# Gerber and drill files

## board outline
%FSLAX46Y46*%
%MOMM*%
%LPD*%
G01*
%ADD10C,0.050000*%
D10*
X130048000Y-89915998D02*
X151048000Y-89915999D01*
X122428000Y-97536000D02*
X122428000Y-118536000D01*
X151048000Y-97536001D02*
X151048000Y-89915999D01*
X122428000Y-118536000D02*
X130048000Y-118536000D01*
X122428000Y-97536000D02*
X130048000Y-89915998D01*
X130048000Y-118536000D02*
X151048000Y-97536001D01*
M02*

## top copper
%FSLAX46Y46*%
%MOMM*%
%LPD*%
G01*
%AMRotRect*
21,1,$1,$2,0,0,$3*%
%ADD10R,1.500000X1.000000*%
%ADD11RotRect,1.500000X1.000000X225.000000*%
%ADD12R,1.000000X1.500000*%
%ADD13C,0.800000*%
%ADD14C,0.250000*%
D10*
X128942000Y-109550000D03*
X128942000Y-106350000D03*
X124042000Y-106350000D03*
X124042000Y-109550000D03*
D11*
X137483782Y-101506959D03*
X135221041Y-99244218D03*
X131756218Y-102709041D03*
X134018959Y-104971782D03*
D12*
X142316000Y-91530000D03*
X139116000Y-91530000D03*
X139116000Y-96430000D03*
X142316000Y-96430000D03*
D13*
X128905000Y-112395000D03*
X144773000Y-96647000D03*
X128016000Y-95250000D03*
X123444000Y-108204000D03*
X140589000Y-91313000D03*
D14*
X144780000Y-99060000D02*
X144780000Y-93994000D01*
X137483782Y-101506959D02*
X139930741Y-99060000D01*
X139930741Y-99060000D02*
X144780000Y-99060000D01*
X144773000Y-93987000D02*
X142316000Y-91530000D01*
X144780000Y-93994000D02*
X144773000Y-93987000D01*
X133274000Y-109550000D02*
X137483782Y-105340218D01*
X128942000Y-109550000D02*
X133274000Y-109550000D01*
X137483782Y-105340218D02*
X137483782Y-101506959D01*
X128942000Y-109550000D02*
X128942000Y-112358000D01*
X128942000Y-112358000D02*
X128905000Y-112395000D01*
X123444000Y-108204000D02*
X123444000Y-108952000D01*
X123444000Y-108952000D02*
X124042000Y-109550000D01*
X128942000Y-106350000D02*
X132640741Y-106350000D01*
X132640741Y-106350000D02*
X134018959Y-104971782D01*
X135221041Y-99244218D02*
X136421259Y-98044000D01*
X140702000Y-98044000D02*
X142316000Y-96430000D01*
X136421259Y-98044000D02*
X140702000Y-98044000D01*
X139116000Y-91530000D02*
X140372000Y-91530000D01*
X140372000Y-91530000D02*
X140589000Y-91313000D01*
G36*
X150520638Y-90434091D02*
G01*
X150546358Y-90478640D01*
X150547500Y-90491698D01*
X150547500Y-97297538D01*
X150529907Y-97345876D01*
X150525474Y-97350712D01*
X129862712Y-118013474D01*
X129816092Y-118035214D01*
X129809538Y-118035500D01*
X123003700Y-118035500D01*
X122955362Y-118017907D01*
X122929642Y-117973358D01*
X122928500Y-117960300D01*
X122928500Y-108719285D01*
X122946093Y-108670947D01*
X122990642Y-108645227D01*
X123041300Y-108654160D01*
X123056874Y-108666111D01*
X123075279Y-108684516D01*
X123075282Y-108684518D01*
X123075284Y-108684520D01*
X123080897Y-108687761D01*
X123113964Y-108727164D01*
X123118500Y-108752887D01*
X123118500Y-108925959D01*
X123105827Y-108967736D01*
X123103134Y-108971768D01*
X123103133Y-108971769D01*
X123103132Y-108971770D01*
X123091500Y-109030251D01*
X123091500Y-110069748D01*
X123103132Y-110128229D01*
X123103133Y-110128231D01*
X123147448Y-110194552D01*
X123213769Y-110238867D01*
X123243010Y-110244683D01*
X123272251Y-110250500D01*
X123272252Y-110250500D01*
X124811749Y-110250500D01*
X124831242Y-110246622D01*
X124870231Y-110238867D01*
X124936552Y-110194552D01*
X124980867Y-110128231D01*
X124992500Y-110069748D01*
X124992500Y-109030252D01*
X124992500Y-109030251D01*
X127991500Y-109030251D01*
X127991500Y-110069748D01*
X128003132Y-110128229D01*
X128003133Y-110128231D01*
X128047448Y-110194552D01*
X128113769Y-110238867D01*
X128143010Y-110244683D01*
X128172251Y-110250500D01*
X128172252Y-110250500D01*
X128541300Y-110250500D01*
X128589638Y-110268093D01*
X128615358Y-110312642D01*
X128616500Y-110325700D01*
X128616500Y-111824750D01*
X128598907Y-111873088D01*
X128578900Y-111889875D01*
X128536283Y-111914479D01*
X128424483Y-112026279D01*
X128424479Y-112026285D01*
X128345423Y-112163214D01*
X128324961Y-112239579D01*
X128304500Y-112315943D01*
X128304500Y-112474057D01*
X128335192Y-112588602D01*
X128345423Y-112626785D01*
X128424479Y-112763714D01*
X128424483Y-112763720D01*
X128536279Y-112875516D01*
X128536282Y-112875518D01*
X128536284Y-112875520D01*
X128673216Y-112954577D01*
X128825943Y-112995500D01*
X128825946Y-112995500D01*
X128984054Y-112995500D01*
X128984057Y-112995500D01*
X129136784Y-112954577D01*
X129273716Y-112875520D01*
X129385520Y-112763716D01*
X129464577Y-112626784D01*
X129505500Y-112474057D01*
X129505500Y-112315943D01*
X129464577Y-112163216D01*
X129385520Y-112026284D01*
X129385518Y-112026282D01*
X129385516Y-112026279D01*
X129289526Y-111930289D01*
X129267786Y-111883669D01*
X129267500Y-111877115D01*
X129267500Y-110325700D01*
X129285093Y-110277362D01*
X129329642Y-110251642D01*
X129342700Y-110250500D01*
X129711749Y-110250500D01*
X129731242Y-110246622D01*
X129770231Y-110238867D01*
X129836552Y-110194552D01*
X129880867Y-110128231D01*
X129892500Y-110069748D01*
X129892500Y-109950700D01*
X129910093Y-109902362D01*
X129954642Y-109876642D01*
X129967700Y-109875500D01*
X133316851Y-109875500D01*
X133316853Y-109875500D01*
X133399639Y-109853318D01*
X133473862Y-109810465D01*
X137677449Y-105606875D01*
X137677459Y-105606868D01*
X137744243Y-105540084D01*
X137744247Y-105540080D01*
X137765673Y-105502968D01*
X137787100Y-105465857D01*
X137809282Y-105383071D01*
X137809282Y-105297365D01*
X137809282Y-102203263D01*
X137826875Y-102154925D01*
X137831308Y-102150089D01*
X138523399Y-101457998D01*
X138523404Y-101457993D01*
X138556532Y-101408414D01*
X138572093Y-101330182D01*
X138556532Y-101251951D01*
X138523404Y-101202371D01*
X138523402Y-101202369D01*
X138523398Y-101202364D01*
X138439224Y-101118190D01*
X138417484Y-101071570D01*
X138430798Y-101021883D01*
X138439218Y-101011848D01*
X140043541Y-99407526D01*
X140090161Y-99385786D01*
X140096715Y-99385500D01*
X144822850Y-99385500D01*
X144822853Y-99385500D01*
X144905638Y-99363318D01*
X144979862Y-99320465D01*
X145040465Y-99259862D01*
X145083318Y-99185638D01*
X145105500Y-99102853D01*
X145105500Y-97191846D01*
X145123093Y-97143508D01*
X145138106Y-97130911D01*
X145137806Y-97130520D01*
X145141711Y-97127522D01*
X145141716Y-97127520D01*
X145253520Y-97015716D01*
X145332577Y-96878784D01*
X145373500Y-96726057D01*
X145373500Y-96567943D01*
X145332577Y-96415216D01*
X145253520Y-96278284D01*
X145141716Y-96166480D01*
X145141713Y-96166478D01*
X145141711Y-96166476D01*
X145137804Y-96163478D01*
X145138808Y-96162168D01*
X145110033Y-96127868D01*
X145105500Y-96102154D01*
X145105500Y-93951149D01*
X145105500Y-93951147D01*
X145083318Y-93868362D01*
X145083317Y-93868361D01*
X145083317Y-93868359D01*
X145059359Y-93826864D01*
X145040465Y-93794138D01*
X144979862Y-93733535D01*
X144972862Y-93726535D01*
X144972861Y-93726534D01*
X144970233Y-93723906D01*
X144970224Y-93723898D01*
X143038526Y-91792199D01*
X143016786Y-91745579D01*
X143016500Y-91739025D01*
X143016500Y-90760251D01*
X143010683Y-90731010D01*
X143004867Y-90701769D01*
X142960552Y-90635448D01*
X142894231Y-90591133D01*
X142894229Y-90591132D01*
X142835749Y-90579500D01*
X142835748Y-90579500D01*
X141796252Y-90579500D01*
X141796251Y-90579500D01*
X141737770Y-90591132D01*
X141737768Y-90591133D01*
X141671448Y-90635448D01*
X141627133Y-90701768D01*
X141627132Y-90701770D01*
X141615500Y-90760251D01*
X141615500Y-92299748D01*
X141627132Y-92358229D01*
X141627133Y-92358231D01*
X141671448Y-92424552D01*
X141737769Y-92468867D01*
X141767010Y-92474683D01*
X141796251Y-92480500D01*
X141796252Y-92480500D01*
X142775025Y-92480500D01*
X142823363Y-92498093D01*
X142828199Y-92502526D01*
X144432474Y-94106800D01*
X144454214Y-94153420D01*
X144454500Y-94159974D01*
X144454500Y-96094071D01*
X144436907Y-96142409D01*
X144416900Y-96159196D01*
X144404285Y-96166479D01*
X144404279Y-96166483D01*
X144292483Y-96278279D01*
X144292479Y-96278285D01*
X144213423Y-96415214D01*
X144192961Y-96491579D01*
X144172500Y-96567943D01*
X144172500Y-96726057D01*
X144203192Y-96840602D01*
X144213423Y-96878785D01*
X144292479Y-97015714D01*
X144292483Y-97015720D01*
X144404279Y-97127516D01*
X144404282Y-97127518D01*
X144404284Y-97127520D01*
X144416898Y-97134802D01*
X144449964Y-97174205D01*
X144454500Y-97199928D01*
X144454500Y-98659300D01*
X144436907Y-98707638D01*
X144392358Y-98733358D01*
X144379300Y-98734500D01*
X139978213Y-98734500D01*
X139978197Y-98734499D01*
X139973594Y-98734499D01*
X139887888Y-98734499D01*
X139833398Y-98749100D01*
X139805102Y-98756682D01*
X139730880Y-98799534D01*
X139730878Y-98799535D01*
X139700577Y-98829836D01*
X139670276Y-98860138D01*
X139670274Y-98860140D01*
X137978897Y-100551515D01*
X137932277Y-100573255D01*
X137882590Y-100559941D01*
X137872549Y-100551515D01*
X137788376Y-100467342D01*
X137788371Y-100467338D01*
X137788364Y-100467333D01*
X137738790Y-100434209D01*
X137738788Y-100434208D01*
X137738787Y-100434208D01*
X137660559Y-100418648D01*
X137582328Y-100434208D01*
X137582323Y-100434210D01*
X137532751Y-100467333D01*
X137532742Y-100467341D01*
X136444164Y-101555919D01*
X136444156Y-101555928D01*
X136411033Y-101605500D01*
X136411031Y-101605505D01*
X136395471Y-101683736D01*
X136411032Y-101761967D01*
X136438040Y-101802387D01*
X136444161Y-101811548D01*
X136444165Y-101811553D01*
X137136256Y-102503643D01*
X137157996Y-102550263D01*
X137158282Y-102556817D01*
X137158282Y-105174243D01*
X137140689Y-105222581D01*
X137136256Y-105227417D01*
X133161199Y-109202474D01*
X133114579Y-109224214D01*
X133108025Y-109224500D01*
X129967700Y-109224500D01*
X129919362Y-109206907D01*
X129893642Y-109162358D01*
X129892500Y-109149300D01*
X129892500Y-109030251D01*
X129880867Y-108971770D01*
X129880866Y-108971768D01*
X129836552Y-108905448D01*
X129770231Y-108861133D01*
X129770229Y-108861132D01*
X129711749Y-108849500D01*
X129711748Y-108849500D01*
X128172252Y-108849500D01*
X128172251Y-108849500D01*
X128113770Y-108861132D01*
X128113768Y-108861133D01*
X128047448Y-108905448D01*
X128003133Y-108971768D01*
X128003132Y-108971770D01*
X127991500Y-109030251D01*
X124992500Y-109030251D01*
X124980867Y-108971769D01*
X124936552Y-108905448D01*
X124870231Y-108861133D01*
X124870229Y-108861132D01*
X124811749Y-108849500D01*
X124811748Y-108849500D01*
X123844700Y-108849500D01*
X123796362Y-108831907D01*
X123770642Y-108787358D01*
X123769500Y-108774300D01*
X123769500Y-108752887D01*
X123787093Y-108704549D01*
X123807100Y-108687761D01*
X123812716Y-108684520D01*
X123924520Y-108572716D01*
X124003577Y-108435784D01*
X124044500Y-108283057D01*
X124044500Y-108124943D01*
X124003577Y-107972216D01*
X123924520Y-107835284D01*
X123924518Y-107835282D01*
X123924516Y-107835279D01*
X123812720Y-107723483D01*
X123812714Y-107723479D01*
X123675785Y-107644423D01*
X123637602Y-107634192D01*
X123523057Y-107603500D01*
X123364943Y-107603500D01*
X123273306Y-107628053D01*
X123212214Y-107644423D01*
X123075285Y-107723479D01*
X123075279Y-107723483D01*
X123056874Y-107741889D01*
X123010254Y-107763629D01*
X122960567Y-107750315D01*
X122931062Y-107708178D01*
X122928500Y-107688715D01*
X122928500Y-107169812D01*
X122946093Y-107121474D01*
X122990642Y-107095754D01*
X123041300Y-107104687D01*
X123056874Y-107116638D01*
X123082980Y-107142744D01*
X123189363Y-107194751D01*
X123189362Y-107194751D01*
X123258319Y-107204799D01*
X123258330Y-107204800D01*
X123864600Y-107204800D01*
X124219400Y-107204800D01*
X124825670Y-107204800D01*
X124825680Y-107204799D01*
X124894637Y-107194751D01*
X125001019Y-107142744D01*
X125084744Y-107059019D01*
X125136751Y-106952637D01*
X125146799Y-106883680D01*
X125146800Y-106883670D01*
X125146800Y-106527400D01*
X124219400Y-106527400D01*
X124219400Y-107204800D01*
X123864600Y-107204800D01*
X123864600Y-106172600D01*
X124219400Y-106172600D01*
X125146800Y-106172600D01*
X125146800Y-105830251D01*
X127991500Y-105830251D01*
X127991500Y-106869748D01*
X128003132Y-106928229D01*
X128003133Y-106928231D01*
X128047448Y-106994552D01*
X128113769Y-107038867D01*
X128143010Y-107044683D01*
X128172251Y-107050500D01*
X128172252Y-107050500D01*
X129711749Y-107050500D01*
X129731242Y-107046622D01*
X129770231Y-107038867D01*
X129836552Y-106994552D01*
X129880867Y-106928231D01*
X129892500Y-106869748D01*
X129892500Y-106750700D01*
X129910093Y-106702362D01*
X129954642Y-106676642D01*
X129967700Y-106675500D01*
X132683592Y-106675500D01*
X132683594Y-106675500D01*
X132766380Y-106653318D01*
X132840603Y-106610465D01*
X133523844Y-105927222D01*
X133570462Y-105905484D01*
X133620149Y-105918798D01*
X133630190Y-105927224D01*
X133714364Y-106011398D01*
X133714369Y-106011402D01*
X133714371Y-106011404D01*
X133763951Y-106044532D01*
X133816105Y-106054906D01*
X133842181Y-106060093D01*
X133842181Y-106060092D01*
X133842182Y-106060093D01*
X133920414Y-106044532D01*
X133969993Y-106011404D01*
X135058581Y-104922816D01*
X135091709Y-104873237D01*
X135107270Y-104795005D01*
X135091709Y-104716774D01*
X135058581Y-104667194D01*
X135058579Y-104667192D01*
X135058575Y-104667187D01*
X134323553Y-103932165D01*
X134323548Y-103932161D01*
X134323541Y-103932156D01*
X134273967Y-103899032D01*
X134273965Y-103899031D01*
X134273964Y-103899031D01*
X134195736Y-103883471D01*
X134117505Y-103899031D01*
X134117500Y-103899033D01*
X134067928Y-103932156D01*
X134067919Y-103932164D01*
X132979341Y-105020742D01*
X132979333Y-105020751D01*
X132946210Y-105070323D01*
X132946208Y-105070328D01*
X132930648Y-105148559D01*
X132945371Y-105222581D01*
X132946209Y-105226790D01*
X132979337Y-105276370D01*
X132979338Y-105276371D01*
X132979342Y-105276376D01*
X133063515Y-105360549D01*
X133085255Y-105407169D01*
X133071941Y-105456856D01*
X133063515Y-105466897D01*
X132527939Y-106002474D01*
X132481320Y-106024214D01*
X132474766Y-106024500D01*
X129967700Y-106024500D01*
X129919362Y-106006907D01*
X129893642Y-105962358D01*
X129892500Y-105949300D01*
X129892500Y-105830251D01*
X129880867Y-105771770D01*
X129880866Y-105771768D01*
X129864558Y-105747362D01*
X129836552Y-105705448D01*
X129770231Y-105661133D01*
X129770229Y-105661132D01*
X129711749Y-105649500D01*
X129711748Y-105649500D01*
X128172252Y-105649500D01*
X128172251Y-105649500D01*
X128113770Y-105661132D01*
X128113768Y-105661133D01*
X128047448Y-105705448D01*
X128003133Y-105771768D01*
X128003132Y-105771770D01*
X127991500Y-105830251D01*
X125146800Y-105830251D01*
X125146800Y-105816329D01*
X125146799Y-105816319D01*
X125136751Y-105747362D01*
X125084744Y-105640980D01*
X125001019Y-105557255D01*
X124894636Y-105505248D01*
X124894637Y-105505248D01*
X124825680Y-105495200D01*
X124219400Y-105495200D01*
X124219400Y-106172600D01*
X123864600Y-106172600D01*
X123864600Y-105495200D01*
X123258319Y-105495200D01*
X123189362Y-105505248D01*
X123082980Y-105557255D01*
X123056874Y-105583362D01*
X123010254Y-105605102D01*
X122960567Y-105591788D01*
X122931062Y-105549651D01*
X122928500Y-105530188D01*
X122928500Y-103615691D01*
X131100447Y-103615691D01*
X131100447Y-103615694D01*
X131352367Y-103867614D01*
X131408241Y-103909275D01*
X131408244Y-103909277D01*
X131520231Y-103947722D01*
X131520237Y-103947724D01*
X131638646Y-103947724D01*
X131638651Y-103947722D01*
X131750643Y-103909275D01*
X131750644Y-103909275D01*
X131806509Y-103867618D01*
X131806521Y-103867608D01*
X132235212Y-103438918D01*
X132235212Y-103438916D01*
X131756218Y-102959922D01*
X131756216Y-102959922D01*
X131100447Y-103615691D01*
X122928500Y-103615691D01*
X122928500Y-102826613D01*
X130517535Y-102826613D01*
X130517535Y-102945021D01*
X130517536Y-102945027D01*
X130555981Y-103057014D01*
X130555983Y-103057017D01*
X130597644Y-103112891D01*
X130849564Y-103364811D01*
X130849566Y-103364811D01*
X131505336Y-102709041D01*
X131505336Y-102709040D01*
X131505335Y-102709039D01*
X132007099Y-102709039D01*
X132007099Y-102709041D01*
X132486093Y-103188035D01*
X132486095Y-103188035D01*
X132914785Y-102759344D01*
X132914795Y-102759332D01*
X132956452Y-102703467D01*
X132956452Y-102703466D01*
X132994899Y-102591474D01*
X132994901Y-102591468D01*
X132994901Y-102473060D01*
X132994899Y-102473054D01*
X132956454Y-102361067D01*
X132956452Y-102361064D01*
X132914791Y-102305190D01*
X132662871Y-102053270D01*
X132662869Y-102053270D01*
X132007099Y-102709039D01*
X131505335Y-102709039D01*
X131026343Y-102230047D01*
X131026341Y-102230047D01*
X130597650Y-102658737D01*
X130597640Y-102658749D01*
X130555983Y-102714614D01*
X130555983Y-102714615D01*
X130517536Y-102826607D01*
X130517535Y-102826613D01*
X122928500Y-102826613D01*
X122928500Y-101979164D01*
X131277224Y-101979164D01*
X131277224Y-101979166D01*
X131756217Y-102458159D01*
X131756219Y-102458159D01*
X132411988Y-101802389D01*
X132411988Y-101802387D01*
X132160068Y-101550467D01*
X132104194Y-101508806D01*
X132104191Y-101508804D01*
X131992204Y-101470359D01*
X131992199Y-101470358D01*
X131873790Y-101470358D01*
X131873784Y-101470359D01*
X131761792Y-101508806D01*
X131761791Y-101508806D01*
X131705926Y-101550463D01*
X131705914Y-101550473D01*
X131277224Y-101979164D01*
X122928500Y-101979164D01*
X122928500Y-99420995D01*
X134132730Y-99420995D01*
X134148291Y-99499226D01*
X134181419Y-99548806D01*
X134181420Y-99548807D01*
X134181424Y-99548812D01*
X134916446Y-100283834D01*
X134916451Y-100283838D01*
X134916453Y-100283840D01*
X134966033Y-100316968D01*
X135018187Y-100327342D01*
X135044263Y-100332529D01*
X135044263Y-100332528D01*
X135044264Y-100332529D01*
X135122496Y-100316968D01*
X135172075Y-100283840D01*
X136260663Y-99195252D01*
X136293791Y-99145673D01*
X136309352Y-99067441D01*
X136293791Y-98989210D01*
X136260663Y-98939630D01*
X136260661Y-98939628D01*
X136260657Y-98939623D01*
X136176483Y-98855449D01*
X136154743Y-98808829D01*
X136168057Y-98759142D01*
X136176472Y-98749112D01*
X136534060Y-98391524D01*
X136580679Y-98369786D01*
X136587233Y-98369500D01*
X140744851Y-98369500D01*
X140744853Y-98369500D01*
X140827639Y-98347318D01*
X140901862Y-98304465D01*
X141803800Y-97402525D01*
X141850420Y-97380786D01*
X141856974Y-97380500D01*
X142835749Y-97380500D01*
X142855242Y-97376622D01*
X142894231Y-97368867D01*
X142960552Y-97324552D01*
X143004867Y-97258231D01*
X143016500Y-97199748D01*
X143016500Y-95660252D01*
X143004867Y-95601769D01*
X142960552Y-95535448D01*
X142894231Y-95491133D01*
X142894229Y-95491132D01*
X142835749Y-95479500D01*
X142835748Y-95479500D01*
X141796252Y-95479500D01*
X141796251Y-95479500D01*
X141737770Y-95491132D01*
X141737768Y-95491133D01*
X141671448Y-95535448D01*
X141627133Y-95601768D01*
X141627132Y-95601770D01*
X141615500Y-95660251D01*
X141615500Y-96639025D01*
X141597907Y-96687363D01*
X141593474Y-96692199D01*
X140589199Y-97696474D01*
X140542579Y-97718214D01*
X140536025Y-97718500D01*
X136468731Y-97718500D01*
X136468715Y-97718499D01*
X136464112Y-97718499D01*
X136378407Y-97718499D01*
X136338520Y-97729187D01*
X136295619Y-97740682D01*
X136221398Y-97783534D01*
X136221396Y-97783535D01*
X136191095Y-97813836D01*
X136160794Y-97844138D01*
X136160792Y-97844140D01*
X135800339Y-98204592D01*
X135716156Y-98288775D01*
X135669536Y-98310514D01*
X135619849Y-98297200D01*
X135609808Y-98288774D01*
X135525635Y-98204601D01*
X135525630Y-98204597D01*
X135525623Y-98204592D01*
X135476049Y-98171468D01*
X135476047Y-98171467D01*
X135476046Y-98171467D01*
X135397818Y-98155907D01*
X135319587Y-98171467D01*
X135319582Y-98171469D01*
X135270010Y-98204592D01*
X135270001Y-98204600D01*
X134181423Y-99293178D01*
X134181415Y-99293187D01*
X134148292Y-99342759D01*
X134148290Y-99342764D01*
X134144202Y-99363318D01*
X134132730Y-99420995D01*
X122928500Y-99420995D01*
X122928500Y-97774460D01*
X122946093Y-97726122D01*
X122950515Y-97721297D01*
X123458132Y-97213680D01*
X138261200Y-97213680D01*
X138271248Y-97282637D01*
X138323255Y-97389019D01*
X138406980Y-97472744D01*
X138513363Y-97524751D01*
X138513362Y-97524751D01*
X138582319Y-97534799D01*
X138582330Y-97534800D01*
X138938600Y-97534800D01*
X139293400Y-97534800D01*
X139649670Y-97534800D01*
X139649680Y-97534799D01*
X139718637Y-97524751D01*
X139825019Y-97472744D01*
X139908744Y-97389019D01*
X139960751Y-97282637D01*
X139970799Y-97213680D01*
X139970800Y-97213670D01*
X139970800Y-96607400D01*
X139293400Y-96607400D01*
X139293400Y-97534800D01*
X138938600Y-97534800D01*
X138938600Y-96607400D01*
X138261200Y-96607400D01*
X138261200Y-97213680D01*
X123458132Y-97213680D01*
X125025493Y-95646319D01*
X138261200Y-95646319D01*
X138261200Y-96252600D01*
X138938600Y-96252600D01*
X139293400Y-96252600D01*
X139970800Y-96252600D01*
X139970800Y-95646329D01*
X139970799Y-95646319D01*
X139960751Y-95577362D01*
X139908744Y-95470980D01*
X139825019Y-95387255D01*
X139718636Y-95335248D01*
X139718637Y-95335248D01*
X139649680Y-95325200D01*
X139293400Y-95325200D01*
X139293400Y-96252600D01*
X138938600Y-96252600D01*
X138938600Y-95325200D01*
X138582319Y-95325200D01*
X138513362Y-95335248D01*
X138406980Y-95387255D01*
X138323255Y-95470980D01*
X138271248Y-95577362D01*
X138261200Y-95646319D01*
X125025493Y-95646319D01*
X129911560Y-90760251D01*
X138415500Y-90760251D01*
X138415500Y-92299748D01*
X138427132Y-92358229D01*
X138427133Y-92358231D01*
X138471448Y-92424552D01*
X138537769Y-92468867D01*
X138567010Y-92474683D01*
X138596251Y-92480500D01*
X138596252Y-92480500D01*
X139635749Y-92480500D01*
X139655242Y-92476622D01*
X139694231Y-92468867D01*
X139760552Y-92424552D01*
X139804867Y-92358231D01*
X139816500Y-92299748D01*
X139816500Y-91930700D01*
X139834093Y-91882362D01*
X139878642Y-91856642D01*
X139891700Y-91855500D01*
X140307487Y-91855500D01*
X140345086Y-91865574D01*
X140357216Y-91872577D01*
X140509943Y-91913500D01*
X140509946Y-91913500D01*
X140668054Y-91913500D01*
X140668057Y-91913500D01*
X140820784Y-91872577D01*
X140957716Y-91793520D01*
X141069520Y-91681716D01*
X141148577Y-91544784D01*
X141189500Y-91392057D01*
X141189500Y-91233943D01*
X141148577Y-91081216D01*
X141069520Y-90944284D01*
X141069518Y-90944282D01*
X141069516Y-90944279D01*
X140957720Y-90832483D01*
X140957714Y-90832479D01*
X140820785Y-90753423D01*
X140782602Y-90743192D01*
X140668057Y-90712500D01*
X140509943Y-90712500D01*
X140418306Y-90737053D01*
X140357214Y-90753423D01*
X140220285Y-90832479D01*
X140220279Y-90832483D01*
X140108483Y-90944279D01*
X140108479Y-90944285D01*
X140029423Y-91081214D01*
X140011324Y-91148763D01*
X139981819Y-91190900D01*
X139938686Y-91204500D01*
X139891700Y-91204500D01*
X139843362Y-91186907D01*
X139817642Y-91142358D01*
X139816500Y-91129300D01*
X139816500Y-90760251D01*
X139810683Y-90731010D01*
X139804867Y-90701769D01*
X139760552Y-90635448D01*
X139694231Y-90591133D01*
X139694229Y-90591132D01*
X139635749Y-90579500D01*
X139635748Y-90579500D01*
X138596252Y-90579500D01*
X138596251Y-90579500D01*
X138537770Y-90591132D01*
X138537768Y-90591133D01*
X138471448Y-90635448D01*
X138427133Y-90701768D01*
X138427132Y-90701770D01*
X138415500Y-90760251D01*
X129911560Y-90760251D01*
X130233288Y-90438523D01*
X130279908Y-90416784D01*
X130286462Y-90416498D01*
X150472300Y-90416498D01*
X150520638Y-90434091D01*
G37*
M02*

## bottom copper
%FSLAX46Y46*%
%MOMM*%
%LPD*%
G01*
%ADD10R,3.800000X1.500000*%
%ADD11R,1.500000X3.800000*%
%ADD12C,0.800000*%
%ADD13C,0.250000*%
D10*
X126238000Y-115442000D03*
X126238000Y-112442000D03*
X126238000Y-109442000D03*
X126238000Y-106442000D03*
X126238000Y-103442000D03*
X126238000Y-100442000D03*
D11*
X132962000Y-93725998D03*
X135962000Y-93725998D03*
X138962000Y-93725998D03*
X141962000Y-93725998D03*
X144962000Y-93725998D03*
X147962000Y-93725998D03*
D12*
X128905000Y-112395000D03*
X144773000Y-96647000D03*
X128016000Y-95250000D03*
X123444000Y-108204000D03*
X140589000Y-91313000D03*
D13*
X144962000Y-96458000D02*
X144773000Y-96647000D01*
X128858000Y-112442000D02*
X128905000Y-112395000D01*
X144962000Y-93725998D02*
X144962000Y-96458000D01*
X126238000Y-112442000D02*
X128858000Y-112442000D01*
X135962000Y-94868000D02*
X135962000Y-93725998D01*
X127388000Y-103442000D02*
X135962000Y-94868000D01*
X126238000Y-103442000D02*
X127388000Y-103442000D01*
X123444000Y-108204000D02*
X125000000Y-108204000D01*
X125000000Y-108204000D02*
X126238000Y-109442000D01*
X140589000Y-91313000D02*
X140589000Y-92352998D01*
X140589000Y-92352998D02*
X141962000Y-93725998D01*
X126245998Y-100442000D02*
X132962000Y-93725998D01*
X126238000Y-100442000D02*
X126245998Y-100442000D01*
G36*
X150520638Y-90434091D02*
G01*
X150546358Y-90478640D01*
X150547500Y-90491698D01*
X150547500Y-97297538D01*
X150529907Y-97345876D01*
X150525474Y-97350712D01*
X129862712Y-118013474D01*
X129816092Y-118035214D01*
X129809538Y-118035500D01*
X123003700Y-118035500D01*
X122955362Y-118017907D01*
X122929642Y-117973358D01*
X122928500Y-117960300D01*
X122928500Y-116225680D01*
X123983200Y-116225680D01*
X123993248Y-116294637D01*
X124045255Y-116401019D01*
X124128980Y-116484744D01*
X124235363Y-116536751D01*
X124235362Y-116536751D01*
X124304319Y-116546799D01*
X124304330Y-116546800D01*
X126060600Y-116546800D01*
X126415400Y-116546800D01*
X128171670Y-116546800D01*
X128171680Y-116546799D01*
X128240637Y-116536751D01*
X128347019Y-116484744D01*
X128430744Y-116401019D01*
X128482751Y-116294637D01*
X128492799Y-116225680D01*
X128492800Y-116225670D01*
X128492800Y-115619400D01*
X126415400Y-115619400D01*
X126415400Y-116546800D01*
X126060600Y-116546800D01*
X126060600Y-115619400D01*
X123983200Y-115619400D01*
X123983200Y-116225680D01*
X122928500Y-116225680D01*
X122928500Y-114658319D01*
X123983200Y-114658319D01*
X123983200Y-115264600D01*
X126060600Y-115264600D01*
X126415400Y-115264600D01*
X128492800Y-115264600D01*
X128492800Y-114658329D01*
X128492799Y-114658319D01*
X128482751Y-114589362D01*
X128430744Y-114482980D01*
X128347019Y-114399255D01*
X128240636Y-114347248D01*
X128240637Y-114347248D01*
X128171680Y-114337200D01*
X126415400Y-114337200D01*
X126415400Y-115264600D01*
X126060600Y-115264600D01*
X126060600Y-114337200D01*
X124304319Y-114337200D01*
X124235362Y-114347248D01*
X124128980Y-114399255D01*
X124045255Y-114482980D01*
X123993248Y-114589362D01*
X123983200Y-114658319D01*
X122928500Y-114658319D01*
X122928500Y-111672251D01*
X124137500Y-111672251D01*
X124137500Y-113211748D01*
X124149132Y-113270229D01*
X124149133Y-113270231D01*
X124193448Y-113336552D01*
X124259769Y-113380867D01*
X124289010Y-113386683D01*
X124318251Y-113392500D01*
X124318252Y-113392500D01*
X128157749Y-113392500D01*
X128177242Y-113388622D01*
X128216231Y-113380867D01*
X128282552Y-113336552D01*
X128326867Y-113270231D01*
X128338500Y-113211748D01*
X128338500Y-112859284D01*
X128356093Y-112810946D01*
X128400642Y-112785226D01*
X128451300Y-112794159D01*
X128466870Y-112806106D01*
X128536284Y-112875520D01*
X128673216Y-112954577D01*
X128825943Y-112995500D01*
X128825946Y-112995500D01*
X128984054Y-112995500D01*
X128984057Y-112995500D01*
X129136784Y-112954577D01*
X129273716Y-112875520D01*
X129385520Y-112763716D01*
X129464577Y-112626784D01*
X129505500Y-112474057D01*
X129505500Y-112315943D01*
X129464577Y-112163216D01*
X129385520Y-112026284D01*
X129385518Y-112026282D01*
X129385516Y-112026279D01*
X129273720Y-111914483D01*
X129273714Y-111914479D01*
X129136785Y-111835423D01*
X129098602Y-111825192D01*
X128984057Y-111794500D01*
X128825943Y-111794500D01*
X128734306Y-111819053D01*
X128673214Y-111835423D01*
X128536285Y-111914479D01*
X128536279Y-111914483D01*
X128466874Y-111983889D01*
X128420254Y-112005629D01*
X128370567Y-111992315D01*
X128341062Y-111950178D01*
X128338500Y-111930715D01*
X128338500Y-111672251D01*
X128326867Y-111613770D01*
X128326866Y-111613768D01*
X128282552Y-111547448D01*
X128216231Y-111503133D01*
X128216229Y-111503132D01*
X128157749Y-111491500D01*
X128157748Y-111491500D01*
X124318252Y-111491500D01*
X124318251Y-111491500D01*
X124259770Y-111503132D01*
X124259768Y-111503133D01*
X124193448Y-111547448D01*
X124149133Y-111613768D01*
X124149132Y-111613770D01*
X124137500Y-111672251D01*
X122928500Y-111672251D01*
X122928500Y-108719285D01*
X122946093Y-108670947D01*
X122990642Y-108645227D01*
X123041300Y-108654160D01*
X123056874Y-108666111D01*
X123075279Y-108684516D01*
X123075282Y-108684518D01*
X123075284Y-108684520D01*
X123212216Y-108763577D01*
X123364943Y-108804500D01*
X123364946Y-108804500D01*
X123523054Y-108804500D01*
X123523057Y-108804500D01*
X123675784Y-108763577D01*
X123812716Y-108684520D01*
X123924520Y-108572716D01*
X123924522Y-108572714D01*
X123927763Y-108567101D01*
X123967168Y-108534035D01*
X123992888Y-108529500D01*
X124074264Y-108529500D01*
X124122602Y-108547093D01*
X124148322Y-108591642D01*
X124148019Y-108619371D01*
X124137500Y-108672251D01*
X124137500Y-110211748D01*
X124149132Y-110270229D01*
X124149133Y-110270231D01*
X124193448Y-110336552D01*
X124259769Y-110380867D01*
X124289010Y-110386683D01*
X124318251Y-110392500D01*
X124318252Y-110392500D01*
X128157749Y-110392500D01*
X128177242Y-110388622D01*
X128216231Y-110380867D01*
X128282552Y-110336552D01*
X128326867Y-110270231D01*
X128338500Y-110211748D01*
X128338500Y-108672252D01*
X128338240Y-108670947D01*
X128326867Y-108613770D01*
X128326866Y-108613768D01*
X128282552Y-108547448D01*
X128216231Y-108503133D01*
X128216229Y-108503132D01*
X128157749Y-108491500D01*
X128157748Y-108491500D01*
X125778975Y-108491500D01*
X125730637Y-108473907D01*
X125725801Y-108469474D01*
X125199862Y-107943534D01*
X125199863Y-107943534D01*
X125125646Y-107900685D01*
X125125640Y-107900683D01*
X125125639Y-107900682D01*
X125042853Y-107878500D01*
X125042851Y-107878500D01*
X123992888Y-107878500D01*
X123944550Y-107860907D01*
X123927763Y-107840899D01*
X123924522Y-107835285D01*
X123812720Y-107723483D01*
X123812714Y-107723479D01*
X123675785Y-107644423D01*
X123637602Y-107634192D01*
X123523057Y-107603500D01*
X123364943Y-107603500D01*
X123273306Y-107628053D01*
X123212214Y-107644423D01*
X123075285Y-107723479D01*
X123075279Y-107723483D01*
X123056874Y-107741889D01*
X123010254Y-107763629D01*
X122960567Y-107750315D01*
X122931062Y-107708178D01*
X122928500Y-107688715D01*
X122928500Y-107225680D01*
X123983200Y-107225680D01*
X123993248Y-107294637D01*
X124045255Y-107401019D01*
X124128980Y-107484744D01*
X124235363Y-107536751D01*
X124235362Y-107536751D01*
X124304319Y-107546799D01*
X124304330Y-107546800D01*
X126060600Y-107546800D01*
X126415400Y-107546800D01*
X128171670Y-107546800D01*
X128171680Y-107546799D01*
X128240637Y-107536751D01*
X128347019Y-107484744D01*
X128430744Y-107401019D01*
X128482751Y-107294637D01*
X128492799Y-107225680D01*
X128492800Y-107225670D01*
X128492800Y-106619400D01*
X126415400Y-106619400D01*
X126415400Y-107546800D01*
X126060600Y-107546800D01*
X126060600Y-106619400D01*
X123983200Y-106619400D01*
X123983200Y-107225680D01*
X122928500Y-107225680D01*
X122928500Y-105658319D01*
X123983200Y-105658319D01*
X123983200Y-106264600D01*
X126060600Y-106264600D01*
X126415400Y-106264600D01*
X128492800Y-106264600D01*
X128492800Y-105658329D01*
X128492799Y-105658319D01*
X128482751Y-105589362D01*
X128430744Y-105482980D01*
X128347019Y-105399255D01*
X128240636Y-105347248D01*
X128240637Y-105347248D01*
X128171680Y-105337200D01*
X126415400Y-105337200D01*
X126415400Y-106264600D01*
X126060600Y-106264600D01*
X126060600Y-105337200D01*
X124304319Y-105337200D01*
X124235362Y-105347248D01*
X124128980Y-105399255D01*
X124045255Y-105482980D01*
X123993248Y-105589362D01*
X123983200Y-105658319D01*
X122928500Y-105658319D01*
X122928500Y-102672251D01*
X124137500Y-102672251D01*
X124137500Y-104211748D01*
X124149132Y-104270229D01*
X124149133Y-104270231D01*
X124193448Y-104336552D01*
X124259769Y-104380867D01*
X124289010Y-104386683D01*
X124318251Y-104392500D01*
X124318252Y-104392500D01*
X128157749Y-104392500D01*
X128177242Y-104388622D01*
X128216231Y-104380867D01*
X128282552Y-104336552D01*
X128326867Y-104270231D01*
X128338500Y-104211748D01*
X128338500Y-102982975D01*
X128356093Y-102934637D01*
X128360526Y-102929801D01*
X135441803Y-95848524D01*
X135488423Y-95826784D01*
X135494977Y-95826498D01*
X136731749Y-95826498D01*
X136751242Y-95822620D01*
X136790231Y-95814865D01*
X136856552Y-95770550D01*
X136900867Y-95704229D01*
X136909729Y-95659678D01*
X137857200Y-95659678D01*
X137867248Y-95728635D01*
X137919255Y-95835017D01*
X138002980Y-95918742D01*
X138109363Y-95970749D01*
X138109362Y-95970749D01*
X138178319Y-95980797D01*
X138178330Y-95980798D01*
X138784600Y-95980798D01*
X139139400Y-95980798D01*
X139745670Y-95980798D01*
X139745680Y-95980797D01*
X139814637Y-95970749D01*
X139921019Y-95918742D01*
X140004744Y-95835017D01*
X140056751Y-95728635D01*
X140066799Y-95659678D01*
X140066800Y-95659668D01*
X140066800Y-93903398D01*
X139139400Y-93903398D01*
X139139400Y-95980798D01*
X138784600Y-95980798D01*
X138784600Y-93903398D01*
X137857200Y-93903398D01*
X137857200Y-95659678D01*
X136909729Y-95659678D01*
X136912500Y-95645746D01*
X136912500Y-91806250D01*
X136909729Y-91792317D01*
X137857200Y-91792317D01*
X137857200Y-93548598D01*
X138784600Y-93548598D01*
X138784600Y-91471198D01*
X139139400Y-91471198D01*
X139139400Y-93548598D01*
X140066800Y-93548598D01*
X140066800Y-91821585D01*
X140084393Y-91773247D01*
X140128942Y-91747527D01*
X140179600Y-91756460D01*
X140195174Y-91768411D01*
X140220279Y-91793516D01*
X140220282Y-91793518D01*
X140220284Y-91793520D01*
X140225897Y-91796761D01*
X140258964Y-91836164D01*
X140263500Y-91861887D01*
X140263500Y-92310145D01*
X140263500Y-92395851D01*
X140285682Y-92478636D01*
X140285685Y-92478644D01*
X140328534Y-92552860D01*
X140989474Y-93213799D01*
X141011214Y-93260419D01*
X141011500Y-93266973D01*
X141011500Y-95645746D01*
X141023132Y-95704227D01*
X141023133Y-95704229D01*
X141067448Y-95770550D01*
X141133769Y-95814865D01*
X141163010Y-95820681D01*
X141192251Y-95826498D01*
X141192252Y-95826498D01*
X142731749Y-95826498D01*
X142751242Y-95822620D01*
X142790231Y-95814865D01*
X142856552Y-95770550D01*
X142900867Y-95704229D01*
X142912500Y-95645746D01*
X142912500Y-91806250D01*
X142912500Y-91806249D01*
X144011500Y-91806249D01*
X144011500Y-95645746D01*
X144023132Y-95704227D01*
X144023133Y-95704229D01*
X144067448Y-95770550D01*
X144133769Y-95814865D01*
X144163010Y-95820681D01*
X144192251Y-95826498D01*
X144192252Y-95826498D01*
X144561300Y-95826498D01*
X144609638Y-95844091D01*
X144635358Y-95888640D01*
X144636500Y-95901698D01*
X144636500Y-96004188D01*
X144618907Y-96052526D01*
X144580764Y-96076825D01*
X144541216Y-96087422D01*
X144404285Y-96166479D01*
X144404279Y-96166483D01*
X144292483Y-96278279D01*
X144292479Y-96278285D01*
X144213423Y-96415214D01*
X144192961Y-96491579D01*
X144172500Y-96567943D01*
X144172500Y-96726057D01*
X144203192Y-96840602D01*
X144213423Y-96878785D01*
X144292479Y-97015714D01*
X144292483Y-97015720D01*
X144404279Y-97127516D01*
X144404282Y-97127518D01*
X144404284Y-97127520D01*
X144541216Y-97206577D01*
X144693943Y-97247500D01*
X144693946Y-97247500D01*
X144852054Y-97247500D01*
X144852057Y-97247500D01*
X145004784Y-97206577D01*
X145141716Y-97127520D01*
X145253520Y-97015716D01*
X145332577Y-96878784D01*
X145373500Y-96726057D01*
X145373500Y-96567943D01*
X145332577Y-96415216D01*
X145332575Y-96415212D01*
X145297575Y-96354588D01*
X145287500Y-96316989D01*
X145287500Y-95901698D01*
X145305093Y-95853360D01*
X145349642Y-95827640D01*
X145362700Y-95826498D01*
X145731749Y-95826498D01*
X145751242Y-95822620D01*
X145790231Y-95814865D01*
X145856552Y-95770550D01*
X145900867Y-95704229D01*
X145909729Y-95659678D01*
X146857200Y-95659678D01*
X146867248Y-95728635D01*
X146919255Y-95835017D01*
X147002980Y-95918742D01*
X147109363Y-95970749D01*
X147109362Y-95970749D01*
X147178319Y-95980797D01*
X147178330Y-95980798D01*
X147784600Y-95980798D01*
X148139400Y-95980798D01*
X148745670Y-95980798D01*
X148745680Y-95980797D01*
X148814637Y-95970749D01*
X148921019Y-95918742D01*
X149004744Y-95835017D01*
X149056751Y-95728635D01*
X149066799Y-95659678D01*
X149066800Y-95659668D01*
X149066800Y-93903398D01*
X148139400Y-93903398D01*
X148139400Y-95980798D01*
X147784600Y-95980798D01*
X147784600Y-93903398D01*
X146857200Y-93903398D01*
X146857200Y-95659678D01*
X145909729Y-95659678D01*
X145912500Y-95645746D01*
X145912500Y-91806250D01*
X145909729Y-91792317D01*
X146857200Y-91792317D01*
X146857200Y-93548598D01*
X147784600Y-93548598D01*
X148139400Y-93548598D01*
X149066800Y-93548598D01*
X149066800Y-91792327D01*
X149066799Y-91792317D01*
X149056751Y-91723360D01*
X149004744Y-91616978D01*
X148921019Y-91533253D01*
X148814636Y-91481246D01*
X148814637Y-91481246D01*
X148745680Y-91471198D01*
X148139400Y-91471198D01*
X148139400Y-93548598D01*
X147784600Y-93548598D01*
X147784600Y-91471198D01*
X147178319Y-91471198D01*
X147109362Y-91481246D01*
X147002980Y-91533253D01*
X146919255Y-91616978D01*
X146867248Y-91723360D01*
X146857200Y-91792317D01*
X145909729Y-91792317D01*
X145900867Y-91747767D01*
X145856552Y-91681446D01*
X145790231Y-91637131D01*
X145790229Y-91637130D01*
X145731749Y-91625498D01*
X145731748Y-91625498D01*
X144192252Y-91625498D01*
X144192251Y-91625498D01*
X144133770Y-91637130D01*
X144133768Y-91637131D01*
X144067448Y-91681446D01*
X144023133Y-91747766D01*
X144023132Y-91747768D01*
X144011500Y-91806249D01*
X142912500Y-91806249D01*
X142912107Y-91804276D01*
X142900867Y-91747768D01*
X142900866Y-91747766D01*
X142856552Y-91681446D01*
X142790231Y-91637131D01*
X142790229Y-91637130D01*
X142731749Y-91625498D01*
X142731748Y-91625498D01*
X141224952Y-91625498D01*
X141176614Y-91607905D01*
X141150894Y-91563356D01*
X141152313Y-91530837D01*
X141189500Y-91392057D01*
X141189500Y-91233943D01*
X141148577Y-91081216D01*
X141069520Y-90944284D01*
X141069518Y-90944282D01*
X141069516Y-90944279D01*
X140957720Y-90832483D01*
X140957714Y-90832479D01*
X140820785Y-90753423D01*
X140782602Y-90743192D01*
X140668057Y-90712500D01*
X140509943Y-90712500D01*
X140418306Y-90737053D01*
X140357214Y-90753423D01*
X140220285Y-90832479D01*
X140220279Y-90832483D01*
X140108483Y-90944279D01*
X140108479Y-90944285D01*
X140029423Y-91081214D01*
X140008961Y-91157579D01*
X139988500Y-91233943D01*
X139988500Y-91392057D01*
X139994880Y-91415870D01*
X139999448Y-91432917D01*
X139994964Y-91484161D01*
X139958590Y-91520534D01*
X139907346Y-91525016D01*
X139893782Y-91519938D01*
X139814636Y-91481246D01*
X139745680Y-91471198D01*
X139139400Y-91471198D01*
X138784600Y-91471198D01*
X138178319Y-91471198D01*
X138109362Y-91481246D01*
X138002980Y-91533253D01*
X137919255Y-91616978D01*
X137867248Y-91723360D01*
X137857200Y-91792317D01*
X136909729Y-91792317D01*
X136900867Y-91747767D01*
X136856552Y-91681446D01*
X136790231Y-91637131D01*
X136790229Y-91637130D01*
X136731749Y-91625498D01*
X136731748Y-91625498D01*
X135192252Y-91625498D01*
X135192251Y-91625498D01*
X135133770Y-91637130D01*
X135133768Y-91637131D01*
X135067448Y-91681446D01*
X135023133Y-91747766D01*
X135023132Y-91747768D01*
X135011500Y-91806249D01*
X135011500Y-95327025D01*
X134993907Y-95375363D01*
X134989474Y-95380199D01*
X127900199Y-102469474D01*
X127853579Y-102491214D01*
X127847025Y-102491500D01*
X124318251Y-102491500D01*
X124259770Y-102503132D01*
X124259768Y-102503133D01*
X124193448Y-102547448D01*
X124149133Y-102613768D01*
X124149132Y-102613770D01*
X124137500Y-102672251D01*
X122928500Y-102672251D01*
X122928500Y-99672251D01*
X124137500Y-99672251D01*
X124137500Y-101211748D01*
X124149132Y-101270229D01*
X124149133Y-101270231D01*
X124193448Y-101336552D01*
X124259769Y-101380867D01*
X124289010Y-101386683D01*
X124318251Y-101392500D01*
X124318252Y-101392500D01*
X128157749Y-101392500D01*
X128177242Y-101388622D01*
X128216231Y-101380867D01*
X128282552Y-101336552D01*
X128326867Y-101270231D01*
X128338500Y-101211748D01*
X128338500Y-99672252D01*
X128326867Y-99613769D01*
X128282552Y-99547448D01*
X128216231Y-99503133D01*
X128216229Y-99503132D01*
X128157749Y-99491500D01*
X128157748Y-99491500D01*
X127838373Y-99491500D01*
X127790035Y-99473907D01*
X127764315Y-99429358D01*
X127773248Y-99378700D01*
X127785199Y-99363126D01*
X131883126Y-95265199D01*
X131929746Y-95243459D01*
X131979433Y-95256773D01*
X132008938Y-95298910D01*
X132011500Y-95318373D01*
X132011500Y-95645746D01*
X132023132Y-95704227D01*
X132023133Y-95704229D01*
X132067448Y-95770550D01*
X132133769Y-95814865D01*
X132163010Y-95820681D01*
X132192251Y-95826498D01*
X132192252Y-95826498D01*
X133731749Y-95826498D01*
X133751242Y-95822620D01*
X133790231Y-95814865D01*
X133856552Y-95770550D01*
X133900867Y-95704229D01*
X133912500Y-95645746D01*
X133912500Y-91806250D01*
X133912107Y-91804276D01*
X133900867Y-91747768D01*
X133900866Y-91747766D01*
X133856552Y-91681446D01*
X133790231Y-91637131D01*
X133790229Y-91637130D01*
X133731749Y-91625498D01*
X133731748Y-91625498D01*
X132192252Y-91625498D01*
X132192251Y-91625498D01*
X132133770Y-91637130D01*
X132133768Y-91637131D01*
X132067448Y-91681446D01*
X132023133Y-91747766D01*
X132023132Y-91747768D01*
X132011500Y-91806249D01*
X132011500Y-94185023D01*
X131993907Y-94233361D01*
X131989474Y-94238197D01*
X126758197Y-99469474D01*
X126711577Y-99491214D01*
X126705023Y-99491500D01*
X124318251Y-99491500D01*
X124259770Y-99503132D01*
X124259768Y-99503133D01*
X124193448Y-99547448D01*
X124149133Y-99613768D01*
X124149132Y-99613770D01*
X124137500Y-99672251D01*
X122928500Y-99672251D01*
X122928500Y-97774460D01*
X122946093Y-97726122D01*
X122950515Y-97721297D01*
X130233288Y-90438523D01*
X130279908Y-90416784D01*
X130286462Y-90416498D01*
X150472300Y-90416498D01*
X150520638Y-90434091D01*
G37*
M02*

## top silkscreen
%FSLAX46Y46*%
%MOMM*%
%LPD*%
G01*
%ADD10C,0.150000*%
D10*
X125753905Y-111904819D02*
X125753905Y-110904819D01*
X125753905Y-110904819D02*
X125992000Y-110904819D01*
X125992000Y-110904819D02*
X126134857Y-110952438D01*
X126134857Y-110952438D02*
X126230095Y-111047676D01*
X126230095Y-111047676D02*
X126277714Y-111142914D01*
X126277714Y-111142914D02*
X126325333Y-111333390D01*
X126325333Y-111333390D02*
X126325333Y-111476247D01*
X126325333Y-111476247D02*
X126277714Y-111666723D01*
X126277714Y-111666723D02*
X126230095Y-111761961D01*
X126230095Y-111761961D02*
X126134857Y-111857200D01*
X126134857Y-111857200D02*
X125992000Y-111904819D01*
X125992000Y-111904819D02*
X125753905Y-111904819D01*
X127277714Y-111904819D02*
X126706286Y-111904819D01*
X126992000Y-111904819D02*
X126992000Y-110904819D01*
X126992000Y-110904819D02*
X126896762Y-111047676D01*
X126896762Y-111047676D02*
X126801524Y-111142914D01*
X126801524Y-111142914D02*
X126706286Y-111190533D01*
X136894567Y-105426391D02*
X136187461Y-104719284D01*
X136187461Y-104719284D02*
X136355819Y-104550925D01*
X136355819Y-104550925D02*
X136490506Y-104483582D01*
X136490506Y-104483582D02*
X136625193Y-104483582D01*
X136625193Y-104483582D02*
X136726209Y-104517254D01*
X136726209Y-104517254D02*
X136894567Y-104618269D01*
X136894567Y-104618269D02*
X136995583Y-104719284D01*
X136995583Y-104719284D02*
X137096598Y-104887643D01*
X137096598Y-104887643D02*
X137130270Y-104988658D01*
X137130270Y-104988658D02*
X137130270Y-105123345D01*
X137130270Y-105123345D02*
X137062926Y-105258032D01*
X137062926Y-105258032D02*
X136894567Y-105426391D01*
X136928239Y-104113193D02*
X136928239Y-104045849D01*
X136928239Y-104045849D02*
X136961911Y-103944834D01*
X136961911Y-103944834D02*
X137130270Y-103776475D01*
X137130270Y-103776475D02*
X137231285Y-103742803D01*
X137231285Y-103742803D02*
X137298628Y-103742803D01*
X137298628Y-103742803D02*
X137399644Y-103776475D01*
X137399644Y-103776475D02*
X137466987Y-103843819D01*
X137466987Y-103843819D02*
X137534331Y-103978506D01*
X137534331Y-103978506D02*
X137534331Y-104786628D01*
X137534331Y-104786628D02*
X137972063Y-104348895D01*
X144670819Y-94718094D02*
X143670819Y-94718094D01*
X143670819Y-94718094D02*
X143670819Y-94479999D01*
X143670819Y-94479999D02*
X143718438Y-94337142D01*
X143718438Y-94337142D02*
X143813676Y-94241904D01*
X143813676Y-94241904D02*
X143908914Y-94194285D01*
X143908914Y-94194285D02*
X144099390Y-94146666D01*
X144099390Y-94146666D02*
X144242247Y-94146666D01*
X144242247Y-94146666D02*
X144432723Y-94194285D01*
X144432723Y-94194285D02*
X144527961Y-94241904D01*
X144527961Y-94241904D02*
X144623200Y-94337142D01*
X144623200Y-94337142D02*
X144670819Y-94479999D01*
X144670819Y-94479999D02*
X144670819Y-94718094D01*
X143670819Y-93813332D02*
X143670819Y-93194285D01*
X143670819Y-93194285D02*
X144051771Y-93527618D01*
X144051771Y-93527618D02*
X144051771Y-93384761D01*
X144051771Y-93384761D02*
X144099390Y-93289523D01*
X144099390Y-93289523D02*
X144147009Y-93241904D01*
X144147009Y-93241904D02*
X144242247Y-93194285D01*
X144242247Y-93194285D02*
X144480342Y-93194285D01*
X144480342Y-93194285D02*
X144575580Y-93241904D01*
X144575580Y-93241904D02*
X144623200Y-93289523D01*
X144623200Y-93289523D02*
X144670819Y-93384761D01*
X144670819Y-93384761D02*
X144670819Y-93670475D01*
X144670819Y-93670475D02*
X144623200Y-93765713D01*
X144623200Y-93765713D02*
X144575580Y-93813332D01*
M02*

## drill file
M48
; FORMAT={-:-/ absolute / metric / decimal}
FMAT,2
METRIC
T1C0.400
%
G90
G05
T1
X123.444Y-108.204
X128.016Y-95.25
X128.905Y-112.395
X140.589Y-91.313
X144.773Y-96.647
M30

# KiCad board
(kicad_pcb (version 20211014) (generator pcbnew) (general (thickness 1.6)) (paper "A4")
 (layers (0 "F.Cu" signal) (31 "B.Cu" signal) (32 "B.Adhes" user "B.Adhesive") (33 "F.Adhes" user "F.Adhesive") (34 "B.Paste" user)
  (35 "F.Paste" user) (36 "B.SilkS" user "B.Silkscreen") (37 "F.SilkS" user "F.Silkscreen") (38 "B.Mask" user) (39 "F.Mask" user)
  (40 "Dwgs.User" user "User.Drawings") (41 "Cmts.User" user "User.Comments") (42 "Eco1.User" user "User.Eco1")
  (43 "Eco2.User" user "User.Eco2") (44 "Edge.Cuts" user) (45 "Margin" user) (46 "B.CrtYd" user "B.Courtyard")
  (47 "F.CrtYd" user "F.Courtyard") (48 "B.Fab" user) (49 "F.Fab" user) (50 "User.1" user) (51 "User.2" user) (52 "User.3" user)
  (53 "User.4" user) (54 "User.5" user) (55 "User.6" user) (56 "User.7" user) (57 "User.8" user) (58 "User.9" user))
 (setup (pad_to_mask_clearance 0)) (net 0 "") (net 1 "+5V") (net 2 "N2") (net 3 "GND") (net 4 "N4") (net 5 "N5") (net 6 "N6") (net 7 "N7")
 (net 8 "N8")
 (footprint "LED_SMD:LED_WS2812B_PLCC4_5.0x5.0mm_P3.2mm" (layer "F.Cu") (at 126.492 107.95 180)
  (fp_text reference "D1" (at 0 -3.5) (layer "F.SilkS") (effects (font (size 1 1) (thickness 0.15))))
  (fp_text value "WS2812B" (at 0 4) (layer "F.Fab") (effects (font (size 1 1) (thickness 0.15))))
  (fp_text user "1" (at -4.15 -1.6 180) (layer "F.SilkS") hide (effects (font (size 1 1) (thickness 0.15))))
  (pad "1" smd rect (at -2.45 -1.6 180) (size 1.5 1) (layers "F.Cu" "F.Paste" "F.Mask") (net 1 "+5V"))
  (pad "2" smd rect (at -2.45 1.6 180) (size 1.5 1) (layers "F.Cu" "F.Paste" "F.Mask") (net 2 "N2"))
  (pad "3" smd rect (at 2.45 1.6 180) (size 1.5 1) (layers "F.Cu" "F.Paste" "F.Mask") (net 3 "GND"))
  (pad "4" smd rect (at 2.45 -1.6 180) (size 1.5 1) (layers "F.Cu" "F.Paste" "F.Mask") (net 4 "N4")))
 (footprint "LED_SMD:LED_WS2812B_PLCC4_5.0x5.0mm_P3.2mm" (layer "F.Cu") (at 134.62 102.108 -135)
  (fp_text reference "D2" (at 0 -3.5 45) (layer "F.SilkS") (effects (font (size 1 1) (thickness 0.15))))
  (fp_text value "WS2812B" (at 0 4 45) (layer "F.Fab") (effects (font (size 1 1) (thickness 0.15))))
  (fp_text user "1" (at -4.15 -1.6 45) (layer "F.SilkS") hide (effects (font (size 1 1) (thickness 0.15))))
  (pad "1" smd rect (at -2.45 -1.6 225) (size 1.5 1) (layers "F.Cu" "F.Paste" "F.Mask") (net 1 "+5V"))
  (pad "2" smd rect (at -2.45 1.6 225) (size 1.5 1) (layers "F.Cu" "F.Paste" "F.Mask") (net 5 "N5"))
  (pad "3" smd rect (at 2.45 1.6 225) (size 1.5 1) (layers "F.Cu" "F.Paste" "F.Mask") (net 3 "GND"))
  (pad "4" smd rect (at 2.45 -1.6 225) (size 1.5 1) (layers "F.Cu" "F.Paste" "F.Mask") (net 2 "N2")))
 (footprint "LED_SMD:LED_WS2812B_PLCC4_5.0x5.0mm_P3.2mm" (layer "F.Cu") (at 140.716 93.98 -90)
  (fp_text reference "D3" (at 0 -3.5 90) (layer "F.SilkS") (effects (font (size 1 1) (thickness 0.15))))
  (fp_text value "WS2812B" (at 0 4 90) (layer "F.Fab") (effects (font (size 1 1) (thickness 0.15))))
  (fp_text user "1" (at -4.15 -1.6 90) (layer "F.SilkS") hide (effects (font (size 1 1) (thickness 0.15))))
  (pad "1" smd rect (at -2.45 -1.6 270) (size 1.5 1) (layers "F.Cu" "F.Paste" "F.Mask") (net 1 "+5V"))
  (pad "2" smd rect (at -2.45 1.6 270) (size 1.5 1) (layers "F.Cu" "F.Paste" "F.Mask") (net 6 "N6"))
  (pad "3" smd rect (at 2.45 1.6 270) (size 1.5 1) (layers "F.Cu" "F.Paste" "F.Mask") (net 3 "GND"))
  (pad "4" smd rect (at 2.45 -1.6 270) (size 1.5 1) (layers "F.Cu" "F.Paste" "F.Mask") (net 5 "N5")))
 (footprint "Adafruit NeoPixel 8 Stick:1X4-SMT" (layer "B.Cu") (at 126.873 107.442 90)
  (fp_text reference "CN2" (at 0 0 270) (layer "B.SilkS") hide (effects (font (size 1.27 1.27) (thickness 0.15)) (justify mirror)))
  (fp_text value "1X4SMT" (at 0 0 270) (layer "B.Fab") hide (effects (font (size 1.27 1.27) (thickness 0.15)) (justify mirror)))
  (pad "1" smd rect (at -8 -0.635 90) (size 1.5 3.8) (layers "B.Cu" "B.Paste" "B.Mask") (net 3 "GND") (solder_mask_margin 0.1016))
  (pad "2" smd rect (at -5 -0.635 90) (size 1.5 3.8) (layers "B.Cu" "B.Paste" "B.Mask") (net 1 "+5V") (solder_mask_margin 0.1016))
  (pad "3" smd rect (at -2 -0.635 90) (size 1.5 3.8) (layers "B.Cu" "B.Paste" "B.Mask") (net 4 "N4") (solder_mask_margin 0.1016))
  (pad "4" smd rect (at 1 -0.635 90) (size 1.5 3.8) (layers "B.Cu" "B.Paste" "B.Mask") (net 3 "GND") (solder_mask_margin 0.1016))
  (pad "5" smd rect (at 4 -0.635 90) (size 1.5 3.8) (layers "B.Cu" "B.Paste" "B.Mask") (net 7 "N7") (solder_mask_margin 0.1016))
  (pad "6" smd rect (at 7 -0.635 90) (size 1.5 3.8) (layers "B.Cu" "B.Paste" "B.Mask") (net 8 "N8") (solder_mask_margin 0.1016)))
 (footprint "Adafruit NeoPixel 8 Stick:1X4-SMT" (layer "B.Cu") (at 140.962 94.360998)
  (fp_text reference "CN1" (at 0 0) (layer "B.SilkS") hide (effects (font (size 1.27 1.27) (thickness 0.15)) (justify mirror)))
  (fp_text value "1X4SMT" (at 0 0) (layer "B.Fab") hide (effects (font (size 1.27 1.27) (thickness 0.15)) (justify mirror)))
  (pad "1" smd rect (at -8 -0.635) (size 1.5 3.8) (layers "B.Cu" "B.Paste" "B.Mask") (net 8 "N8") (solder_mask_margin 0.1016))
  (pad "2" smd rect (at -5 -0.635) (size 1.5 3.8) (layers "B.Cu" "B.Paste" "B.Mask") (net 7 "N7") (solder_mask_margin 0.1016))
  (pad "3" smd rect (at -2 -0.635) (size 1.5 3.8) (layers "B.Cu" "B.Paste" "B.Mask") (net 3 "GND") (solder_mask_margin 0.1016))
  (pad "4" smd rect (at 1 -0.635) (size 1.5 3.8) (layers "B.Cu" "B.Paste" "B.Mask") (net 6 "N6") (solder_mask_margin 0.1016))
  (pad "5" smd rect (at 4 -0.635) (size 1.5 3.8) (layers "B.Cu" "B.Paste" "B.Mask") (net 1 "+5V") (solder_mask_margin 0.1016))
  (pad "6" smd rect (at 7 -0.635) (size 1.5 3.8) (layers "B.Cu" "B.Paste" "B.Mask") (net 3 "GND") (solder_mask_margin 0.1016)))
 (gr_line (start 130.048 89.915998) (end 151.048 89.915999) (layer "Edge.Cuts") (width 0.05))
 (gr_line (start 122.428 97.536) (end 122.428 118.536) (layer "Edge.Cuts") (width 0.05))
 (gr_line locked (start 151.048 97.536001) (end 151.048 89.915999) (layer "Edge.Cuts") (width 0.05))
 (gr_line locked (start 122.428 118.536) (end 130.048 118.536) (layer "Edge.Cuts") (width 0.05))
 (gr_line (start 122.428 97.536) (end 130.048 89.915998) (layer "Edge.Cuts") (width 0.05))
 (gr_line (start 130.048 118.536) (end 151.048 97.536001) (layer "Edge.Cuts") (width 0.05))
 (segment (start 144.78 99.06) (end 144.78 93.994) (width 0.25) (layer "F.Cu") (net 1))
 (segment (start 137.483782 101.506959) (end 139.930741 99.06) (width 0.25) (layer "F.Cu") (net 1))
 (segment (start 139.930741 99.06) (end 144.78 99.06) (width 0.25) (layer "F.Cu") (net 1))
 (segment (start 144.773 93.987) (end 142.316 91.53) (width 0.25) (layer "F.Cu") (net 1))
 (segment (start 144.78 93.994) (end 144.773 93.987) (width 0.25) (layer "F.Cu") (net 1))
 (segment (start 133.274 109.55) (end 137.483782 105.340218) (width 0.25) (layer "F.Cu") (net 1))
 (segment (start 128.942 109.55) (end 133.274 109.55) (width 0.25) (layer "F.Cu") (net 1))
 (segment (start 137.483782 105.340218) (end 137.483782 101.506959) (width 0.25) (layer "F.Cu") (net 1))
 (segment (start 128.942 109.55) (end 128.942 112.358) (width 0.25) (layer "F.Cu") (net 1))
 (segment (start 128.942 112.358) (end 128.905 112.395) (width 0.25) (layer "F.Cu") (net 1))
 (via (at 128.905 112.395) (size 0.8) (drill 0.4) (layers "F.Cu" "B.Cu") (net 1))
 (via (at 144.773 96.647) (size 0.8) (drill 0.4) (layers "F.Cu" "B.Cu") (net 1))
 (segment (start 144.962 96.458) (end 144.773 96.647) (width 0.25) (layer "B.Cu") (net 1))
 (segment (start 128.858 112.442) (end 128.905 112.395) (width 0.25) (layer "B.Cu") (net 1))
 (segment (start 144.962 93.725998) (end 144.962 96.458) (width 0.25) (layer "B.Cu") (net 1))
 (segment (start 126.238 112.442) (end 128.858 112.442) (width 0.25) (layer "B.Cu") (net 1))
 (via (at 128.016 95.25) (size 0.8) (drill 0.4) (layers "F.Cu" "B.Cu") (free) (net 3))
 (segment (start 135.962 94.868) (end 135.962 93.725998) (width 0.25) (layer "B.Cu") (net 7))
 (segment (start 127.388 103.442) (end 135.962 94.868) (width 0.25) (layer "B.Cu") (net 7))
 (segment (start 126.238 103.442) (end 127.388 103.442) (width 0.25) (layer "B.Cu") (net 7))
 (segment (start 123.444 108.204) (end 123.444 108.952) (width 0.25) (layer "F.Cu") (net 4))
 (segment (start 123.444 108.952) (end 124.042 109.55) (width 0.25) (layer "F.Cu") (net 4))
 (via (at 123.444 108.204) (size 0.8) (drill 0.4) (layers "F.Cu" "B.Cu") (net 4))
 (segment (start 123.444 108.204) (end 125 108.204) (width 0.25) (layer "B.Cu") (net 4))
 (segment (start 125 108.204) (end 126.238 109.442) (width 0.25) (layer "B.Cu") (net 4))
 (segment (start 128.942 106.35) (end 132.640741 106.35) (width 0.25) (layer "F.Cu") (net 2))
 (segment (start 132.640741 106.35) (end 134.018959 104.971782) (width 0.25) (layer "F.Cu") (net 2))
 (segment (start 135.221041 99.244218) (end 136.421259 98.044) (width 0.25) (layer "F.Cu") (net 5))
 (segment (start 140.702 98.044) (end 142.316 96.43) (width 0.25) (layer "F.Cu") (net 5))
 (segment (start 136.421259 98.044) (end 140.702 98.044) (width 0.25) (layer "F.Cu") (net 5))
 (segment (start 139.116 91.53) (end 140.372 91.53) (width 0.25) (layer "F.Cu") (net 6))
 (segment (start 140.372 91.53) (end 140.589 91.313) (width 0.25) (layer "F.Cu") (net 6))
 (via (at 140.589 91.313) (size 0.8) (drill 0.4) (layers "F.Cu" "B.Cu") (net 6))
 (segment (start 140.589 91.313) (end 140.589 92.352998) (width 0.25) (layer "B.Cu") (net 6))
 (segment (start 140.589 92.352998) (end 141.962 93.725998) (width 0.25) (layer "B.Cu") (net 6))
 (segment (start 126.245998 100.442) (end 132.962 93.725998) (width 0.25) (layer "B.Cu") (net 8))
 (segment (start 126.238 100.442) (end 126.245998 100.442) (width 0.25) (layer "B.Cu") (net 8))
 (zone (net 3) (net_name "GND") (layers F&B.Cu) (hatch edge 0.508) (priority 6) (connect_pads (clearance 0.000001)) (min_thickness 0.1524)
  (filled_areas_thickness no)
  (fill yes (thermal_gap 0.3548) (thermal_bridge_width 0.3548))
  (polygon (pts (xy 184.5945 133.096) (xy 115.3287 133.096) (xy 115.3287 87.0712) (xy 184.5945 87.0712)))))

